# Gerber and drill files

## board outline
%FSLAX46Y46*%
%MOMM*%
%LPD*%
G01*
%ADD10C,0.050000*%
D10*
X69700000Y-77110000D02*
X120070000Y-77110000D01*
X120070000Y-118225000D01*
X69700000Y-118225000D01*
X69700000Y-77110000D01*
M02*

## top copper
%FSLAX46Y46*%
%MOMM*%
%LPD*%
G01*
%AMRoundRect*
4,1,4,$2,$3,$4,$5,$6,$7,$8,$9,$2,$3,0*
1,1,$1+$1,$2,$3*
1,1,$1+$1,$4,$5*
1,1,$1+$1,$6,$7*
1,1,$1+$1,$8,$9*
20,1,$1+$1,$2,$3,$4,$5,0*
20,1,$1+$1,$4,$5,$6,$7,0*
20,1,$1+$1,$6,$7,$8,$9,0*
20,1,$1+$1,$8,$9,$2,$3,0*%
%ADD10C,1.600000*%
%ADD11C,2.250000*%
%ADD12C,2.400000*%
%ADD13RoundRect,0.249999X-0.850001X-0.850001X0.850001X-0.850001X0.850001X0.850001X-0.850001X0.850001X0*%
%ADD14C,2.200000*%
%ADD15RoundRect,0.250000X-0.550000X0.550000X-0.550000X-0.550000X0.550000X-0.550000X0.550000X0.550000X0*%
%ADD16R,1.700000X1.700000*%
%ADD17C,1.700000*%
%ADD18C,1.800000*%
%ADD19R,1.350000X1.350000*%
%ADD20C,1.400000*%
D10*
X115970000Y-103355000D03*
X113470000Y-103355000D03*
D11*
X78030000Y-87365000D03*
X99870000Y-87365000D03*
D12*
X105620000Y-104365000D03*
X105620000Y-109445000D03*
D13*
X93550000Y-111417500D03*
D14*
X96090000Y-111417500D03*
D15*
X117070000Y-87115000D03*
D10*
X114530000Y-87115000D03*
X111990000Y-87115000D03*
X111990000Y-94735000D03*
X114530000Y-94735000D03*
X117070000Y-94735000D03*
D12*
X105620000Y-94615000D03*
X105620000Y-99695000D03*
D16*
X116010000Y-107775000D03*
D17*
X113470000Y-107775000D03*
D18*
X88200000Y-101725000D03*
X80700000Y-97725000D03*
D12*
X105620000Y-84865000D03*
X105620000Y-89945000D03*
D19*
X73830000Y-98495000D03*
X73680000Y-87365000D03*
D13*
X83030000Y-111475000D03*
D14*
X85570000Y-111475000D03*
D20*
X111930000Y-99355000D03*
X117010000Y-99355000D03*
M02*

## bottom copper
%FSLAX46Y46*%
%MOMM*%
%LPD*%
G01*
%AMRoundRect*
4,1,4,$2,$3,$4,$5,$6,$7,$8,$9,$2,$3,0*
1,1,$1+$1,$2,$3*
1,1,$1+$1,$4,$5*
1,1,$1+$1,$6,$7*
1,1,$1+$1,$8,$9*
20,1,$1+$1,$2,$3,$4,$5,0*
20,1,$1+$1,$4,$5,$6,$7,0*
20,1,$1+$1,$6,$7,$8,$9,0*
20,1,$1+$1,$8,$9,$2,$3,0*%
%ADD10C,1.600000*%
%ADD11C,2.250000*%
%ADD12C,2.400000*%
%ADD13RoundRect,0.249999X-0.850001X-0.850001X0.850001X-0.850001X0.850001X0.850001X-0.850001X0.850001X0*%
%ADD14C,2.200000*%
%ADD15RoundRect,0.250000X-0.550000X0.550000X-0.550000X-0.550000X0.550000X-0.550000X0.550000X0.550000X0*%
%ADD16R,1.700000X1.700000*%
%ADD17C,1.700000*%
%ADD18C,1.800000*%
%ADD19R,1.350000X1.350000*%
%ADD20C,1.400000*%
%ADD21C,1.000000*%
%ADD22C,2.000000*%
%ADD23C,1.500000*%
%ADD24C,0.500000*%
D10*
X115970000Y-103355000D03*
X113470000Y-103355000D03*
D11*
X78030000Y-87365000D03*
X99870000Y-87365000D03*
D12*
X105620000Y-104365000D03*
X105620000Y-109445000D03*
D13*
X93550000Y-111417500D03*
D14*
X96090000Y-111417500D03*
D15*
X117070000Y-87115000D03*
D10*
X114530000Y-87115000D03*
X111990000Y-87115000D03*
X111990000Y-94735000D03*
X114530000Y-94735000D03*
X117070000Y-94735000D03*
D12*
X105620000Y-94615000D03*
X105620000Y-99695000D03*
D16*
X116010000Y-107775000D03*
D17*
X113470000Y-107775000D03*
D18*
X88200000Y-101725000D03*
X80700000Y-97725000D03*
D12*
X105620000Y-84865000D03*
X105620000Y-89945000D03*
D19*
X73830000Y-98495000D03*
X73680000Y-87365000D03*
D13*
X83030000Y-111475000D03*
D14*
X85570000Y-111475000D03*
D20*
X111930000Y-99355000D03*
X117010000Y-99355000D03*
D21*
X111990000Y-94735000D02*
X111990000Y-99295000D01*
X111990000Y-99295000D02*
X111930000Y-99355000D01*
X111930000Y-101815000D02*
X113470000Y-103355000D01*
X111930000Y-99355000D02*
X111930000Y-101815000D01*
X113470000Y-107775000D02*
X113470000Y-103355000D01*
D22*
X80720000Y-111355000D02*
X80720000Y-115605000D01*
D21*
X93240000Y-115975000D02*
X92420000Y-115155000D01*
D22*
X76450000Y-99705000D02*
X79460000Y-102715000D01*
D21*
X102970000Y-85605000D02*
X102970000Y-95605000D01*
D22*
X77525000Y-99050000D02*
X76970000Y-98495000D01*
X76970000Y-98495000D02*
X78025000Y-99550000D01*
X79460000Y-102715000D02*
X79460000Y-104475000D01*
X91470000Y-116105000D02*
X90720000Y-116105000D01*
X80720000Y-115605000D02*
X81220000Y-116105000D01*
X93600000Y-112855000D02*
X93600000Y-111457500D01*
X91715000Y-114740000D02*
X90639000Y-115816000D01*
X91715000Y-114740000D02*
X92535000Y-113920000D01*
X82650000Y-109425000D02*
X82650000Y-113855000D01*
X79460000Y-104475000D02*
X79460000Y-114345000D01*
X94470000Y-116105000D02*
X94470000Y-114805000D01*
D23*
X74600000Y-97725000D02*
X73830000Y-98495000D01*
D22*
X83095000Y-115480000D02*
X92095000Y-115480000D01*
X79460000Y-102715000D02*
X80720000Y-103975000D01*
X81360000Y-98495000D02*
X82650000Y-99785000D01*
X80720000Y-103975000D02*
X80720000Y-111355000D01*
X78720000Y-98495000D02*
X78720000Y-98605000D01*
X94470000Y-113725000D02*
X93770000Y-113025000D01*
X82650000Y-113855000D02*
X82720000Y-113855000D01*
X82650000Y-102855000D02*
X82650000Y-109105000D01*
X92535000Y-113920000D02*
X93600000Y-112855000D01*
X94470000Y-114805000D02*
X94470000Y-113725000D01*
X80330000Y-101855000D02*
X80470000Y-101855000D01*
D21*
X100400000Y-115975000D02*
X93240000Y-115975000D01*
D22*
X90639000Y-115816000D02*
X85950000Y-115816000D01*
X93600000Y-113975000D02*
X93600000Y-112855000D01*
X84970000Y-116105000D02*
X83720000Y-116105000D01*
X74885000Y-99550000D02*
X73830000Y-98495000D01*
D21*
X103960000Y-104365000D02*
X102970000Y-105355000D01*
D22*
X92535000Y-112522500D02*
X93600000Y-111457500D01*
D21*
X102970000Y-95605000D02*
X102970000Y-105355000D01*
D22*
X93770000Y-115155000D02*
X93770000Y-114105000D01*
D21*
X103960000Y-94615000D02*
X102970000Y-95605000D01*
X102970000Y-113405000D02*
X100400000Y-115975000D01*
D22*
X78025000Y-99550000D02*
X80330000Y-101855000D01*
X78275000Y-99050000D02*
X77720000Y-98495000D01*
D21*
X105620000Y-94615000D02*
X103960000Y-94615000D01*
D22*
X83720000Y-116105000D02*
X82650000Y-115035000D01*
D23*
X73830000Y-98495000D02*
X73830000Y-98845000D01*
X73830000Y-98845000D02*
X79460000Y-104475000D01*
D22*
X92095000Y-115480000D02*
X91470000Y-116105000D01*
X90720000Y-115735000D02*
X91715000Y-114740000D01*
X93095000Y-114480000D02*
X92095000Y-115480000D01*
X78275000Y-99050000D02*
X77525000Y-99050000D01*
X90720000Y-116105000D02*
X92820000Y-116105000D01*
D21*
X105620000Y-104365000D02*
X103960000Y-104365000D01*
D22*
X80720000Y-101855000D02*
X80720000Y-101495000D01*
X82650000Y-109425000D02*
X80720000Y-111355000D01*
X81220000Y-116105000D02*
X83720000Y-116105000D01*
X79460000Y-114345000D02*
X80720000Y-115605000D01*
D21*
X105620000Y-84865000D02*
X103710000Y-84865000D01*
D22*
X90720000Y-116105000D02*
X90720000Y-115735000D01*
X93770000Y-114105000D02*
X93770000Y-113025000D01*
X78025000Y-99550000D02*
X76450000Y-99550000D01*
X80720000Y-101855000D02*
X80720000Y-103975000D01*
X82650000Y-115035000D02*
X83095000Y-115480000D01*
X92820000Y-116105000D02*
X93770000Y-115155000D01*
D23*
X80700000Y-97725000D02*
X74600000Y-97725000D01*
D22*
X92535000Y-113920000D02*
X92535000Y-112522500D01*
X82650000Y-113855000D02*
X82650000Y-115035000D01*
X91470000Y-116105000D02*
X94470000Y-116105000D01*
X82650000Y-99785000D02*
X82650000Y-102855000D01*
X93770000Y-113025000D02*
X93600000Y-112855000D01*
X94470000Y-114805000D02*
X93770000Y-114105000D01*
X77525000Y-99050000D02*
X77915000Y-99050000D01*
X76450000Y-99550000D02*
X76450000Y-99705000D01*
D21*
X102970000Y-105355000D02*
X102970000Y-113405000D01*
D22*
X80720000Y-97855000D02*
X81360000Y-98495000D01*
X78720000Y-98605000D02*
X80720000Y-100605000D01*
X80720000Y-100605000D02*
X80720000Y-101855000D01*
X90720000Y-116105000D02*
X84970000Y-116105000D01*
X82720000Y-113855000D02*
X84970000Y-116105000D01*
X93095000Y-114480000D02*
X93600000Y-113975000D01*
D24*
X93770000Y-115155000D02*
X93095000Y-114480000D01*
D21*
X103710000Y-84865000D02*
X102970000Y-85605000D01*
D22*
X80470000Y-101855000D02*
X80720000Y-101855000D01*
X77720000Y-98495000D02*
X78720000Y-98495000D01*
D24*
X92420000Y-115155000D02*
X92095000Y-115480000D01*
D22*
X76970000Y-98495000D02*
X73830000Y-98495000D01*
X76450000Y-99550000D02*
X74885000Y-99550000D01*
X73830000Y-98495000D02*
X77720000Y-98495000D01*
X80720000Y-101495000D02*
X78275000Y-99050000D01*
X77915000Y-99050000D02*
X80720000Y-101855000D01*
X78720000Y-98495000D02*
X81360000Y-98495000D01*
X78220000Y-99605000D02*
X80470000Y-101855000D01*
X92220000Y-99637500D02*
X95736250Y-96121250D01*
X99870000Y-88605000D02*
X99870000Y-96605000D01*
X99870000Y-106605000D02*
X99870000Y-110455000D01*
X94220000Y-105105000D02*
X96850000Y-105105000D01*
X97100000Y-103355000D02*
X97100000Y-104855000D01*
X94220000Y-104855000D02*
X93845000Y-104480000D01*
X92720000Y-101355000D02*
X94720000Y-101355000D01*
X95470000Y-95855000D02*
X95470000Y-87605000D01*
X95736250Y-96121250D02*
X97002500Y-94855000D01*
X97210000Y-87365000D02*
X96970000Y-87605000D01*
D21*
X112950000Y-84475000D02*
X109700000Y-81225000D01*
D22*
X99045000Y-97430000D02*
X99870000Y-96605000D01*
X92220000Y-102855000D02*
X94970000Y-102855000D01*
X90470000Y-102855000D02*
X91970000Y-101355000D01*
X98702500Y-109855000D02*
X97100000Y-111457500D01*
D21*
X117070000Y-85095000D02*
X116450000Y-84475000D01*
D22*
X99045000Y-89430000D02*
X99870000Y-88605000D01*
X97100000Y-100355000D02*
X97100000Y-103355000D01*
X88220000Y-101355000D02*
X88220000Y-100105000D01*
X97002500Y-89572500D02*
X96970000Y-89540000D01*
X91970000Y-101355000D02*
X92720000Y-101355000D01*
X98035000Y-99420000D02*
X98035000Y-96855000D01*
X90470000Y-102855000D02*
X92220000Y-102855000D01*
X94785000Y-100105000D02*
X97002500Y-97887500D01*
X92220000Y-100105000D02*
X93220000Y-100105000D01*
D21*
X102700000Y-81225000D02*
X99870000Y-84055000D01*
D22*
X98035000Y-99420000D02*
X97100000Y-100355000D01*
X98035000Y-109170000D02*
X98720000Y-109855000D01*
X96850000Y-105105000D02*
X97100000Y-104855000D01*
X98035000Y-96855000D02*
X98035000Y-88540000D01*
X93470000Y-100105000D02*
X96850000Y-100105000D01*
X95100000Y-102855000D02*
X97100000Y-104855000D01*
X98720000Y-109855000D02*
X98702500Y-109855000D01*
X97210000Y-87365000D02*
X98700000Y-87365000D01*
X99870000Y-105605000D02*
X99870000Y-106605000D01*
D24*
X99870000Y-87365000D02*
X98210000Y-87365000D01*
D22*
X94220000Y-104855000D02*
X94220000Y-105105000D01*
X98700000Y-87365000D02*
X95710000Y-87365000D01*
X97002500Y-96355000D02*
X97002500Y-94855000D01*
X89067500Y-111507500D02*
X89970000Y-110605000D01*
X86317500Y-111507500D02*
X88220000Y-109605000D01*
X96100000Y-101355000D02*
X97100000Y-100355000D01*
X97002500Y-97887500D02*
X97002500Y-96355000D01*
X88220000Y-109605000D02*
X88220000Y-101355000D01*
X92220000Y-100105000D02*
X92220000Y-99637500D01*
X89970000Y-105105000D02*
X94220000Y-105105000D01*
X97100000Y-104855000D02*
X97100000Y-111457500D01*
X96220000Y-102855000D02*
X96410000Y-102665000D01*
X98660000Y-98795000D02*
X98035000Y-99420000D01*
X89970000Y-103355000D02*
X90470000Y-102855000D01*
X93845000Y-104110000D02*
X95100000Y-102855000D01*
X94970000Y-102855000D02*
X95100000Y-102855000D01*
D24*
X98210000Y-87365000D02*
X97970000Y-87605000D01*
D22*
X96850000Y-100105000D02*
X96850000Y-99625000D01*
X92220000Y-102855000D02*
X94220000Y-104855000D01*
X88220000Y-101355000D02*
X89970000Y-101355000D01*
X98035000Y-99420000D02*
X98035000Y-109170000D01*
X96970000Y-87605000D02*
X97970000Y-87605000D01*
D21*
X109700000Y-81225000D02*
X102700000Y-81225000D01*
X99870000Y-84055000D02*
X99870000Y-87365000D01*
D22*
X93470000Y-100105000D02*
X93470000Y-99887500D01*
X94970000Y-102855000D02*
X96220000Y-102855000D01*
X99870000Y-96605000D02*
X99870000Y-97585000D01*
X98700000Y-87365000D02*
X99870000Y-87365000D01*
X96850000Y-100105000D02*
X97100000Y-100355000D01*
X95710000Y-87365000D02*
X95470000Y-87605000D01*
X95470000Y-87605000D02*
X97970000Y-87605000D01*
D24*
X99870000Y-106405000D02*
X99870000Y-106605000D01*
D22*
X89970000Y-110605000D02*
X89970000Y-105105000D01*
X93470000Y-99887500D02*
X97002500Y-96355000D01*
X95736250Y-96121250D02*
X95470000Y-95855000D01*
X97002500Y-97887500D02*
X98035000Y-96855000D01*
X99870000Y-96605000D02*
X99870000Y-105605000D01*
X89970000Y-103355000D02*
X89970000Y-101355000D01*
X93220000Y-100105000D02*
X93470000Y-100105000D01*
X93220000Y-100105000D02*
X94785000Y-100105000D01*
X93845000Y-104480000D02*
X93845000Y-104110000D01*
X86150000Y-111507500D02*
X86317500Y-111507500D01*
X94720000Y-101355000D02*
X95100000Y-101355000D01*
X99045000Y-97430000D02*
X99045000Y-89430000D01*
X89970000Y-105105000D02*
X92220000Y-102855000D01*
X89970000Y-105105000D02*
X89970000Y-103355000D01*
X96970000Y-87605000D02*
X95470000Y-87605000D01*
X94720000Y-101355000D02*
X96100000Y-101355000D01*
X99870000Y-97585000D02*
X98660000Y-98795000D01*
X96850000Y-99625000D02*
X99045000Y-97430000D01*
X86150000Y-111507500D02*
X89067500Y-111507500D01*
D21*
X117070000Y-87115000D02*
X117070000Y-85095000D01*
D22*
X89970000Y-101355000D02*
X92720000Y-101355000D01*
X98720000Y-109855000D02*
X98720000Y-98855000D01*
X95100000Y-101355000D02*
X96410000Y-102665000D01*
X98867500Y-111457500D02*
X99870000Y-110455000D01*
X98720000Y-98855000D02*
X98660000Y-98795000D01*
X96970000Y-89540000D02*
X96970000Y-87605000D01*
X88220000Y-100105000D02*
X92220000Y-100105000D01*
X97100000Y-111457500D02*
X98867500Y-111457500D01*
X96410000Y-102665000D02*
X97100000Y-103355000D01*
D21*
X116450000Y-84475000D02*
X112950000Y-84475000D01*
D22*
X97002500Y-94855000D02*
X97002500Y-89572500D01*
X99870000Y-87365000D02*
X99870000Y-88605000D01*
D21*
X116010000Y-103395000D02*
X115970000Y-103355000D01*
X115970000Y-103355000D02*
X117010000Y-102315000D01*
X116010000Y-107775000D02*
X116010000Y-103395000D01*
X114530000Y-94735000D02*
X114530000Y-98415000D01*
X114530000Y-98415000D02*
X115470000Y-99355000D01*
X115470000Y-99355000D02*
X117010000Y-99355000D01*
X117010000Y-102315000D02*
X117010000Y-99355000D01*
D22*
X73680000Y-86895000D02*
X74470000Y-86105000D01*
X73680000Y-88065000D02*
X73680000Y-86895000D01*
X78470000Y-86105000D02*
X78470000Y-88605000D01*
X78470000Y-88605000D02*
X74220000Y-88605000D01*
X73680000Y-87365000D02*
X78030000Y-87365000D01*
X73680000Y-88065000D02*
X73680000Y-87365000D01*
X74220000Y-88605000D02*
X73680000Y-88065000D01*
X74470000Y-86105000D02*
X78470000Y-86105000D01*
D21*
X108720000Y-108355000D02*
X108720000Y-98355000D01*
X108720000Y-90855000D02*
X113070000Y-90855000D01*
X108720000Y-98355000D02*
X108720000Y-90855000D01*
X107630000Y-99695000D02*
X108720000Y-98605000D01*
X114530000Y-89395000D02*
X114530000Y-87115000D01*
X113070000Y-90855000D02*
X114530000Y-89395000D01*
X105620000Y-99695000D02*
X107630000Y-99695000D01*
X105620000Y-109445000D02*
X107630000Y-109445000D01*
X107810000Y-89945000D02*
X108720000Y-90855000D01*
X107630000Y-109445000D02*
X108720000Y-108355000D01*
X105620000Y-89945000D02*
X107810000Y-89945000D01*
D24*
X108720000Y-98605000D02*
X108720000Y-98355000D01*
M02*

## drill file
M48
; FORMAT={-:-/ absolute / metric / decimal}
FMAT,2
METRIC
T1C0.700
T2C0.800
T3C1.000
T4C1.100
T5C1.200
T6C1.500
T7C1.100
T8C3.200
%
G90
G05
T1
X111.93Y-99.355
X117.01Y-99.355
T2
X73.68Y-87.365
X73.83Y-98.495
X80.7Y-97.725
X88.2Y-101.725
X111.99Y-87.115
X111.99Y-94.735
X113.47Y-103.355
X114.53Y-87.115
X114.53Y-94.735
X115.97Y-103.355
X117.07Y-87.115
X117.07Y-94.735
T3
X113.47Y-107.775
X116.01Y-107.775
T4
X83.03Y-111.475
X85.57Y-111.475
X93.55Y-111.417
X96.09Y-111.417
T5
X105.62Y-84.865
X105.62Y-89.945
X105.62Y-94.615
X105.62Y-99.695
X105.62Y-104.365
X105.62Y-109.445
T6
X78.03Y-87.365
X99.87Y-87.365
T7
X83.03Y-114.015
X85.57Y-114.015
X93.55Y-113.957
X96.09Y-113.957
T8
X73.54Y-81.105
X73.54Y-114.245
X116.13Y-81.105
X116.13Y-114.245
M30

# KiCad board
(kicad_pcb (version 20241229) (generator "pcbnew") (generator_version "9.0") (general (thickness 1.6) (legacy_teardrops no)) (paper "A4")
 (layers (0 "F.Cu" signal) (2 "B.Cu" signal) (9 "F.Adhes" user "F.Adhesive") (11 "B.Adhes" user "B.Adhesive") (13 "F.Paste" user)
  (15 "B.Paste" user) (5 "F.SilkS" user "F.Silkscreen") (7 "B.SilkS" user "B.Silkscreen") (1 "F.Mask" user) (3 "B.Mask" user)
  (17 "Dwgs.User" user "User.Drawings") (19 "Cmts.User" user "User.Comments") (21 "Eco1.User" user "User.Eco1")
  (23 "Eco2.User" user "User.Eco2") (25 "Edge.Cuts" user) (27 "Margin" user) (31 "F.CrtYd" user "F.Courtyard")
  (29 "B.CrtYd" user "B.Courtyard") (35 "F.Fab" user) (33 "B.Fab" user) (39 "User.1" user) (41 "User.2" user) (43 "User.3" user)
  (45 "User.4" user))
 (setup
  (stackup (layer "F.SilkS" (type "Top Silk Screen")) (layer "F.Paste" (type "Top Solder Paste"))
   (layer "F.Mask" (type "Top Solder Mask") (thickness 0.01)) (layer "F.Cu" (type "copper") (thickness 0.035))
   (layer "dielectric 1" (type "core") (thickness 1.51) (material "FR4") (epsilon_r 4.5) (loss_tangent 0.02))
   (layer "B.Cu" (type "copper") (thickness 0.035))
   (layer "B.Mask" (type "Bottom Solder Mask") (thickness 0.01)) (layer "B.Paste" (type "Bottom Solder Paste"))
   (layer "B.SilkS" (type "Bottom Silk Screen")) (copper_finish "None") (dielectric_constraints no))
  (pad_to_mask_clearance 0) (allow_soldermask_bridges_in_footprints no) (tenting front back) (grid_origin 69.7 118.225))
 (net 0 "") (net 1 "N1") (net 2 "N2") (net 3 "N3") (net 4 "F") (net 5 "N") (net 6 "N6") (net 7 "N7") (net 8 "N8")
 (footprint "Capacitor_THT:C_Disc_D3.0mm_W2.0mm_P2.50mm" (layer "F.Cu") (at 115.97 103.355 180)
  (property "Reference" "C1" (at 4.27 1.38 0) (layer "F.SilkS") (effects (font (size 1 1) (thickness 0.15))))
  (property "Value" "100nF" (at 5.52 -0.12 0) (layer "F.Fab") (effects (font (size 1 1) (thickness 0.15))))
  (pad "1" thru_hole circle (at 0 0 180) (size 1.6 1.6) (drill 0.8) (layers "*.Cu" "*.Mask") (remove_unused_layers no) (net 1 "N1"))
  (pad "2" thru_hole circle (at 2.5 0 180) (size 1.6 1.6) (drill 0.8) (layers "*.Cu" "*.Mask") (remove_unused_layers no) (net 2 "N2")))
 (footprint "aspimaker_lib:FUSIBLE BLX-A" (layer "F.Cu") (at 88.95 87.365)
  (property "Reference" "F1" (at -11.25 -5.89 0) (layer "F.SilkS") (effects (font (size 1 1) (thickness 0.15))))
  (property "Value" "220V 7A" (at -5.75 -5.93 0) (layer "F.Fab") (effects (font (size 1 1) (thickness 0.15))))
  (pad "1" thru_hole circle (at -10.92 0) (size 2.25 2.25) (drill 1.5) (layers "*.Cu" "*.Mask") (remove_unused_layers no) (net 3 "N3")
   (solder_mask_margin 0.102))
  (pad "2" thru_hole circle (at 10.92 0) (size 2.25 2.25) (drill 1.5) (layers "*.Cu" "*.Mask") (remove_unused_layers no) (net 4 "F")
   (solder_mask_margin 0.102)))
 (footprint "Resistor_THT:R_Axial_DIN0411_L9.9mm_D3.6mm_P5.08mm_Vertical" (layer "F.Cu") (at 105.62 104.365 -90)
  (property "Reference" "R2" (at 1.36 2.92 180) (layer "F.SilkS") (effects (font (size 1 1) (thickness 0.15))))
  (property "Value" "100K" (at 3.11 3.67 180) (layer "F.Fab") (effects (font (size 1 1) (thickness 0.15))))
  (pad "1" thru_hole circle (at 0 0 270) (size 2.4 2.4) (drill 1.2) (layers "*.Cu" "*.Mask") (remove_unused_layers no) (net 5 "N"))
  (pad "2" thru_hole circle (at 5.08 0 270) (size 2.4 2.4) (drill 1.2) (layers "*.Cu" "*.Mask") (remove_unused_layers no) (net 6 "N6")))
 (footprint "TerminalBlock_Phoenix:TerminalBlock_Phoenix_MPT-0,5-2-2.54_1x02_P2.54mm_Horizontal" (layer "F.Cu") (at 93.55 111.4175)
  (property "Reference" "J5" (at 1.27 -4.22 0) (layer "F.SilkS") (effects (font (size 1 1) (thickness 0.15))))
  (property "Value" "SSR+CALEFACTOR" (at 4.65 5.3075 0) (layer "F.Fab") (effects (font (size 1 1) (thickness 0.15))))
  (pad "" np_thru_hole circle (at 0 2.54) (size 1.1 1.1) (drill 1.1) (layers "*.Cu" "*.Mask"))
  (pad "" np_thru_hole circle (at 2.54 2.54) (size 1.1 1.1) (drill 1.1) (layers "*.Cu" "*.Mask"))
  (pad "1" thru_hole roundrect (at 0 0) (size 2.2 2.2) (drill 1.1) (layers "*.Cu" "*.Mask") (remove_unused_layers no)
   (roundrect_rratio 0.113636) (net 5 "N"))
  (pad "2" thru_hole circle (at 2.54 0) (size 2.2 2.2) (drill 1.1) (layers "*.Cu" "*.Mask") (remove_unused_layers no) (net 4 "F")))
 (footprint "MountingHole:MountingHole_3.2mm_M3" (layer "F.Cu") (at 116.13 114.245)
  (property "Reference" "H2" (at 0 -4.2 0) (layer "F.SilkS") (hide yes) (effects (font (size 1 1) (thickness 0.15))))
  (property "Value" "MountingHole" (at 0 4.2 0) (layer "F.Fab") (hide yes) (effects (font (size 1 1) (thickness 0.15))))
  (pad "" np_thru_hole circle (at 0 0) (size 3.2 3.2) (drill 3.2) (layers "*.Cu" "*.Mask")))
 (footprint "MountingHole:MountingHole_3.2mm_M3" (layer "F.Cu") (at 73.54 81.105)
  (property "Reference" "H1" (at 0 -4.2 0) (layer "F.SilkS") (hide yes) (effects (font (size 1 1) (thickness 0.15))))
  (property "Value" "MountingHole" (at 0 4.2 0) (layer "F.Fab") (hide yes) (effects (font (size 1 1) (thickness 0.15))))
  (pad "" np_thru_hole circle (at 0 0) (size 3.2 3.2) (drill 3.2) (layers "*.Cu" "*.Mask")))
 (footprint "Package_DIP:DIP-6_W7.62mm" (layer "F.Cu") (at 117.07 87.115 -90)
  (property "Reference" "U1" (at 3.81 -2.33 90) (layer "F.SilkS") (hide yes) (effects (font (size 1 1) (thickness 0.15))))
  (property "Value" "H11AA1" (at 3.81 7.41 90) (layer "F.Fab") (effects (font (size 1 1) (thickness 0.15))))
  (pad "1" thru_hole roundrect (at 0 0 270) (size 1.6 1.6) (drill 0.8) (layers "*.Cu" "*.Mask") (remove_unused_layers no)
   (roundrect_rratio 0.15625) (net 4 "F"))
  (pad "2" thru_hole circle (at 0 2.54 270) (size 1.6 1.6) (drill 0.8) (layers "*.Cu" "*.Mask") (remove_unused_layers no) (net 6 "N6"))
  (pad "3" thru_hole circle (at 0 5.08 270) (size 1.6 1.6) (drill 0.8) (layers "*.Cu" "*.Mask") (remove_unused_layers no) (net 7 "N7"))
  (pad "4" thru_hole circle (at 7.62 5.08 270) (size 1.6 1.6) (drill 0.8) (layers "*.Cu" "*.Mask") (remove_unused_layers no) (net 2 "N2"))
  (pad "5" thru_hole circle (at 7.62 2.54 270) (size 1.6 1.6) (drill 0.8) (layers "*.Cu" "*.Mask") (remove_unused_layers no) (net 1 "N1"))
  (pad "6" thru_hole circle (at 7.62 0 270) (size 1.6 1.6) (drill 0.8) (layers "*.Cu" "*.Mask") (remove_unused_layers no) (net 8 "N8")))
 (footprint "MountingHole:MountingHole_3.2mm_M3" (layer "F.Cu") (at 116.13 81.105)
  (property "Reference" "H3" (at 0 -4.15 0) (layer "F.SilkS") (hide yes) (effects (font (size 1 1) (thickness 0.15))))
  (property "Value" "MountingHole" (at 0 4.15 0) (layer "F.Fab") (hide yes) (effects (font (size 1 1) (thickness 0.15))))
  (pad "" np_thru_hole circle (at 0 0) (size 3.2 3.2) (drill 3.2) (layers "*.Cu" "*.Mask")))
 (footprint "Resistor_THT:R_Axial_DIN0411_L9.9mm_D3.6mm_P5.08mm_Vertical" (layer "F.Cu") (at 105.62 94.615 -90)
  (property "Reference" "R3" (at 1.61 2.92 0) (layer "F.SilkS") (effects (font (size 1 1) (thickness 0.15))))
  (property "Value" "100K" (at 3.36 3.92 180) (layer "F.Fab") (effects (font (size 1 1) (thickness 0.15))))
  (pad "1" thru_hole circle (at 0 0 270) (size 2.4 2.4) (drill 1.2) (layers "*.Cu" "*.Mask") (remove_unused_layers no) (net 5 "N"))
  (pad "2" thru_hole circle (at 5.08 0 270) (size 2.4 2.4) (drill 1.2) (layers "*.Cu" "*.Mask") (remove_unused_layers no) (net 6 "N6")))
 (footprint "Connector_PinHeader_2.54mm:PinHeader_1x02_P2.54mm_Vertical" (layer "F.Cu") (at 116.01 107.775 -90)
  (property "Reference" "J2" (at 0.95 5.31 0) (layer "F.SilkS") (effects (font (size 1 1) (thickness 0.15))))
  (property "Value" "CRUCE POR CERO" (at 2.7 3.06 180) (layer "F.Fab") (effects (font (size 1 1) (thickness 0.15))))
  (pad "1" thru_hole rect (at 0 0 270) (size 1.7 1.7) (drill 1) (layers "*.Cu" "*.Mask") (remove_unused_layers no) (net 1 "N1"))
  (pad "2" thru_hole circle (at 0 2.54 270) (size 1.7 1.7) (drill 1) (layers "*.Cu" "*.Mask") (remove_unused_layers no) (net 2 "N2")))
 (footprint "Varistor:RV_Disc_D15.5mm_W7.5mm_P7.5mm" (layer "F.Cu") (at 88.2 101.725 180)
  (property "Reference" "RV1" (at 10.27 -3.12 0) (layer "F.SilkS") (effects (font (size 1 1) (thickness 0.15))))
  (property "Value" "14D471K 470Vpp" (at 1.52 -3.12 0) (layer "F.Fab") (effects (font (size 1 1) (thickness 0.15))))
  (pad "1" thru_hole circle (at 0 0 180) (size 1.8 1.8) (drill 0.8) (layers "*.Cu" "*.Mask") (remove_unused_layers no) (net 4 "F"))
  (pad "2" thru_hole circle (at 7.5 4 180) (size 1.8 1.8) (drill 0.8) (layers "*.Cu" "*.Mask") (remove_unused_layers no) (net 5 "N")))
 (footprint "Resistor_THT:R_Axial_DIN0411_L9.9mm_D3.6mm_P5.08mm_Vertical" (layer "F.Cu") (at 105.62 84.865 -90)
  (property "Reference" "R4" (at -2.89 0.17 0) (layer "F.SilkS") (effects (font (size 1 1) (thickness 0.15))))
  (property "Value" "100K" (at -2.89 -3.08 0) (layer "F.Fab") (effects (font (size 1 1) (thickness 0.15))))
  (pad "1" thru_hole circle (at 0 0 270) (size 2.4 2.4) (drill 1.2) (layers "*.Cu" "*.Mask") (remove_unused_layers no) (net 5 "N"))
  (pad "2" thru_hole circle (at 5.08 0 270) (size 2.4 2.4) (drill 1.2) (layers "*.Cu" "*.Mask") (remove_unused_layers no) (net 6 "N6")))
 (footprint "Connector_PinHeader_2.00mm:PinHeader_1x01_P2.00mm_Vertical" (layer "F.Cu") (at 73.83 98.495)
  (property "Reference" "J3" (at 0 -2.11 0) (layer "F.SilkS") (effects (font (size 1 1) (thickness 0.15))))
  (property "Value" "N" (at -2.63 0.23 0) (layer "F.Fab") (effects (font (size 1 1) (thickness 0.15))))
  (pad "1" thru_hole rect (at 0 0) (size 1.35 1.35) (drill 0.8) (layers "*.Cu" "*.Mask") (remove_unused_layers no) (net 5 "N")))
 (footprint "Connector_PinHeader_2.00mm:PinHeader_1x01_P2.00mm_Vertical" (layer "F.Cu") (at 73.68 87.365)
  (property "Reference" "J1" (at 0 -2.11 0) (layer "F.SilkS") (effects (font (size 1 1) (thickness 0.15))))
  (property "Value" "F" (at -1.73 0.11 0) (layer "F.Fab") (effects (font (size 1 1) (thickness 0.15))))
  (pad "1" thru_hole rect (at 0 0) (size 1.35 1.35) (drill 0.8) (layers "*.Cu" "*.Mask") (remove_unused_layers no) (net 3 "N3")))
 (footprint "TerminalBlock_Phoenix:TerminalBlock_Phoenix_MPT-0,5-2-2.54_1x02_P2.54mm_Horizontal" (layer "F.Cu") (at 83.03 111.475)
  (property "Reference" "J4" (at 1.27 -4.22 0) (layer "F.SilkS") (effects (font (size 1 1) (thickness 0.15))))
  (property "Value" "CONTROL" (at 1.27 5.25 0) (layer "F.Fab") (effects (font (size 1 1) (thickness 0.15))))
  (pad "" np_thru_hole circle (at 0 2.54) (size 1.1 1.1) (drill 1.1) (layers "*.Cu" "*.Mask"))
  (pad "" np_thru_hole circle (at 2.54 2.54) (size 1.1 1.1) (drill 1.1) (layers "*.Cu" "*.Mask"))
  (pad "1" thru_hole roundrect (at 0 0) (size 2.2 2.2) (drill 1.1) (layers "*.Cu" "*.Mask") (remove_unused_layers no)
   (roundrect_rratio 0.113636) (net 5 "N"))
  (pad "2" thru_hole circle (at 2.54 0) (size 2.2 2.2) (drill 1.1) (layers "*.Cu" "*.Mask") (remove_unused_layers no) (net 4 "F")))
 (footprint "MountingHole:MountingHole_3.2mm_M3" (layer "F.Cu") (at 73.54 114.245)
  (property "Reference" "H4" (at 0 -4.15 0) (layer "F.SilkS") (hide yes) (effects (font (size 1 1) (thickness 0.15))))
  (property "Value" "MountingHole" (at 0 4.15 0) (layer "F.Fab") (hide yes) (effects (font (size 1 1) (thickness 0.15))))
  (pad "" np_thru_hole circle (at 0 0) (size 3.2 3.2) (drill 3.2) (layers "*.Cu" "*.Mask")))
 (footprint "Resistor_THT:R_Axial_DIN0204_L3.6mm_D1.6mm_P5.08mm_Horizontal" (layer "F.Cu") (at 111.93 99.355)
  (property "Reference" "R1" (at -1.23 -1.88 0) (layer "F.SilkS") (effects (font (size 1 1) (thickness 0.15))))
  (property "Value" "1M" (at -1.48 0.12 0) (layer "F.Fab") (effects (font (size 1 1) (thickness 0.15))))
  (pad "1" thru_hole circle (at 0 0) (size 1.4 1.4) (drill 0.7) (layers "*.Cu" "*.Mask") (remove_unused_layers no) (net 2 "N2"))
  (pad "2" thru_hole circle (at 5.08 0) (size 1.4 1.4) (drill 0.7) (layers "*.Cu" "*.Mask") (remove_unused_layers no) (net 1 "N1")))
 (gr_rect (start 69.7 77.11) (end 120.07 118.225) (stroke (width 0.05) (type solid)) (fill no) (layer "Edge.Cuts"))
 (segment (start 111.99 94.735) (end 111.99 99.295) (width 1) (layer "B.Cu") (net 2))
 (segment (start 111.99 99.295) (end 111.93 99.355) (width 1) (layer "B.Cu") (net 2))
 (segment (start 111.93 101.815) (end 113.47 103.355) (width 1) (layer "B.Cu") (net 2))
 (segment (start 111.93 99.355) (end 111.93 101.815) (width 1) (layer "B.Cu") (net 2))
 (segment (start 113.47 107.775) (end 113.47 103.355) (width 1) (layer "B.Cu") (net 2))
 (segment (start 80.72 111.355) (end 80.72 115.605) (width 2) (layer "B.Cu") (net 5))
 (segment (start 93.24 115.975) (end 92.42 115.155) (width 1) (layer "B.Cu") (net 5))
 (segment (start 76.45 99.705) (end 79.46 102.715) (width 2) (layer "B.Cu") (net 5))
 (segment (start 102.97 85.605) (end 102.97 95.605) (width 1) (layer "B.Cu") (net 5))
 (segment (start 77.525 99.05) (end 76.97 98.495) (width 2) (layer "B.Cu") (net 5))
 (segment (start 76.97 98.495) (end 78.025 99.55) (width 2) (layer "B.Cu") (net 5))
 (segment (start 79.46 102.715) (end 79.46 104.475) (width 2) (layer "B.Cu") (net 5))
 (segment (start 91.47 116.105) (end 90.72 116.105) (width 2) (layer "B.Cu") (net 5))
 (segment (start 80.72 115.605) (end 81.22 116.105) (width 2) (layer "B.Cu") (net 5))
 (segment (start 93.6 112.855) (end 93.6 111.4575) (width 2) (layer "B.Cu") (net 5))
 (segment (start 91.715 114.74) (end 90.639 115.816) (width 2) (layer "B.Cu") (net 5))
 (segment (start 91.715 114.74) (end 92.535 113.92) (width 2) (layer "B.Cu") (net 5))
 (segment (start 82.65 109.425) (end 82.65 113.855) (width 2) (layer "B.Cu") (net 5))
 (segment (start 79.46 104.475) (end 79.46 114.345) (width 2) (layer "B.Cu") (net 5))
 (segment (start 94.47 116.105) (end 94.47 114.805) (width 2) (layer "B.Cu") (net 5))
 (segment (start 74.6 97.725) (end 73.83 98.495) (width 1.5) (layer "B.Cu") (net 5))
 (segment (start 83.095 115.48) (end 92.095 115.48) (width 2) (layer "B.Cu") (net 5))
 (segment (start 79.46 102.715) (end 80.72 103.975) (width 2) (layer "B.Cu") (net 5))
 (segment (start 81.36 98.495) (end 82.65 99.785) (width 2) (layer "B.Cu") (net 5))
 (segment (start 80.72 103.975) (end 80.72 111.355) (width 2) (layer "B.Cu") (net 5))
 (segment (start 78.72 98.495) (end 78.72 98.605) (width 2) (layer "B.Cu") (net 5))
 (segment (start 94.47 113.725) (end 93.77 113.025) (width 2) (layer "B.Cu") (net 5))
 (segment (start 82.65 113.855) (end 82.72 113.855) (width 2) (layer "B.Cu") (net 5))
 (segment (start 82.65 102.855) (end 82.65 109.105) (width 2) (layer "B.Cu") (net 5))
 (segment (start 92.535 113.92) (end 93.6 112.855) (width 2) (layer "B.Cu") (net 5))
 (segment (start 94.47 114.805) (end 94.47 113.725) (width 2) (layer "B.Cu") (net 5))
 (segment (start 80.33 101.855) (end 80.47 101.855) (width 2) (layer "B.Cu") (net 5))
 (segment (start 100.4 115.975) (end 93.24 115.975) (width 1) (layer "B.Cu") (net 5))
 (segment (start 90.639 115.816) (end 85.95 115.816) (width 2) (layer "B.Cu") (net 5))
 (segment (start 93.6 113.975) (end 93.6 112.855) (width 2) (layer "B.Cu") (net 5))
 (segment (start 84.97 116.105) (end 83.72 116.105) (width 2) (layer "B.Cu") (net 5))
 (segment (start 74.885 99.55) (end 73.83 98.495) (width 2) (layer "B.Cu") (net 5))
 (segment (start 103.96 104.365) (end 102.97 105.355) (width 1) (layer "B.Cu") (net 5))
 (segment (start 92.535 112.5225) (end 93.6 111.4575) (width 2) (layer "B.Cu") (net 5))
 (segment (start 102.97 95.605) (end 102.97 105.355) (width 1) (layer "B.Cu") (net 5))
 (segment (start 93.77 115.155) (end 93.77 114.105) (width 2) (layer "B.Cu") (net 5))
 (segment (start 103.96 94.615) (end 102.97 95.605) (width 1) (layer "B.Cu") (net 5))
 (segment (start 102.97 113.405) (end 100.4 115.975) (width 1) (layer "B.Cu") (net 5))
 (segment (start 78.025 99.55) (end 80.33 101.855) (width 2) (layer "B.Cu") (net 5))
 (segment (start 78.275 99.05) (end 77.72 98.495) (width 2) (layer "B.Cu") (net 5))
 (segment (start 105.62 94.615) (end 103.96 94.615) (width 1) (layer "B.Cu") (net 5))
 (segment (start 83.72 116.105) (end 82.65 115.035) (width 2) (layer "B.Cu") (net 5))
 (segment (start 73.83 98.495) (end 73.83 98.845) (width 1.5) (layer "B.Cu") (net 5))
 (segment (start 73.83 98.845) (end 79.46 104.475) (width 1.5) (layer "B.Cu") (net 5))
 (segment (start 92.095 115.48) (end 91.47 116.105) (width 2) (layer "B.Cu") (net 5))
 (segment (start 90.72 115.735) (end 91.715 114.74) (width 2) (layer "B.Cu") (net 5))
 (segment (start 93.095 114.48) (end 92.095 115.48) (width 2) (layer "B.Cu") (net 5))
 (segment (start 78.275 99.05) (end 77.525 99.05) (width 2) (layer "B.Cu") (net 5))
 (segment (start 90.72 116.105) (end 92.82 116.105) (width 2) (layer "B.Cu") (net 5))
 (segment (start 105.62 104.365) (end 103.96 104.365) (width 1) (layer "B.Cu") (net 5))
 (segment (start 80.72 101.855) (end 80.72 101.495) (width 2) (layer "B.Cu") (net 5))
 (segment (start 82.65 109.425) (end 80.72 111.355) (width 2) (layer "B.Cu") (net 5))
 (segment (start 81.22 116.105) (end 83.72 116.105) (width 2) (layer "B.Cu") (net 5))
 (segment (start 79.46 114.345) (end 80.72 115.605) (width 2) (layer "B.Cu") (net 5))
 (segment (start 105.62 84.865) (end 103.71 84.865) (width 1) (layer "B.Cu") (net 5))
 (segment (start 90.72 116.105) (end 90.72 115.735) (width 2) (layer "B.Cu") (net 5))
 (segment (start 93.77 114.105) (end 93.77 113.025) (width 2) (layer "B.Cu") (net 5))
 (segment (start 78.025 99.55) (end 76.45 99.55) (width 2) (layer "B.Cu") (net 5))
 (segment (start 80.72 101.855) (end 80.72 103.975) (width 2) (layer "B.Cu") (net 5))
 (segment (start 82.65 115.035) (end 83.095 115.48) (width 2) (layer "B.Cu") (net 5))
 (segment (start 92.82 116.105) (end 93.77 115.155) (width 2) (layer "B.Cu") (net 5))
 (segment (start 80.7 97.725) (end 74.6 97.725) (width 1.5) (layer "B.Cu") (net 5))
 (segment (start 92.535 113.92) (end 92.535 112.5225) (width 2) (layer "B.Cu") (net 5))
 (segment (start 82.65 113.855) (end 82.65 115.035) (width 2) (layer "B.Cu") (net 5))
 (segment (start 91.47 116.105) (end 94.47 116.105) (width 2) (layer "B.Cu") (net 5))
 (segment (start 82.65 99.785) (end 82.65 102.855) (width 2) (layer "B.Cu") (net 5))
 (segment (start 93.77 113.025) (end 93.6 112.855) (width 2) (layer "B.Cu") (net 5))
 (segment (start 94.47 114.805) (end 93.77 114.105) (width 2) (layer "B.Cu") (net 5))
 (segment (start 77.525 99.05) (end 77.915 99.05) (width 2) (layer "B.Cu") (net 5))
 (segment (start 76.45 99.55) (end 76.45 99.705) (width 2) (layer "B.Cu") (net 5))
 (segment (start 102.97 105.355) (end 102.97 113.405) (width 1) (layer "B.Cu") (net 5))
 (segment (start 80.72 97.855) (end 81.36 98.495) (width 2) (layer "B.Cu") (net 5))
 (segment (start 78.72 98.605) (end 80.72 100.605) (width 2) (layer "B.Cu") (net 5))
 (segment (start 80.72 100.605) (end 80.72 101.855) (width 2) (layer "B.Cu") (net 5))
 (segment (start 90.72 116.105) (end 84.97 116.105) (width 2) (layer "B.Cu") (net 5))
 (segment (start 82.72 113.855) (end 84.97 116.105) (width 2) (layer "B.Cu") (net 5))
 (segment (start 93.095 114.48) (end 93.6 113.975) (width 2) (layer "B.Cu") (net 5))
 (segment (start 93.77 115.155) (end 93.095 114.48) (width 0.5) (layer "B.Cu") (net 5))
 (segment (start 103.71 84.865) (end 102.97 85.605) (width 1) (layer "B.Cu") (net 5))
 (segment (start 80.47 101.855) (end 80.72 101.855) (width 2) (layer "B.Cu") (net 5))
 (segment (start 77.72 98.495) (end 78.72 98.495) (width 2) (layer "B.Cu") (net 5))
 (segment (start 92.42 115.155) (end 92.095 115.48) (width 0.5) (layer "B.Cu") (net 5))
 (segment (start 76.97 98.495) (end 73.83 98.495) (width 2) (layer "B.Cu") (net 5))
 (segment (start 76.45 99.55) (end 74.885 99.55) (width 2) (layer "B.Cu") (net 5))
 (segment (start 73.83 98.495) (end 77.72 98.495) (width 2) (layer "B.Cu") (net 5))
 (segment (start 80.72 101.495) (end 78.275 99.05) (width 2) (layer "B.Cu") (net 5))
 (segment (start 77.915 99.05) (end 80.72 101.855) (width 2) (layer "B.Cu") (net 5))
 (segment (start 78.72 98.495) (end 81.36 98.495) (width 2) (layer "B.Cu") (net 5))
 (segment (start 78.22 99.605) (end 80.47 101.855) (width 2) (layer "B.Cu") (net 5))
 (segment (start 92.22 99.6375) (end 95.73625 96.12125) (width 2) (layer "B.Cu") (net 4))
 (segment (start 99.87 88.605) (end 99.87 96.605) (width 2) (layer "B.Cu") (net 4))
 (segment (start 99.87 106.605) (end 99.87 110.455) (width 2) (layer "B.Cu") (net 4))
 (segment (start 94.22 105.105) (end 96.85 105.105) (width 2) (layer "B.Cu") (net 4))
 (segment (start 97.1 103.355) (end 97.1 104.855) (width 2) (layer "B.Cu") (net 4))
 (segment (start 94.22 104.855) (end 93.845 104.48) (width 2) (layer "B.Cu") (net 4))
 (segment (start 92.72 101.355) (end 94.72 101.355) (width 2) (layer "B.Cu") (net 4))
 (segment (start 95.47 95.855) (end 95.47 87.605) (width 2) (layer "B.Cu") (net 4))
 (segment (start 95.73625 96.12125) (end 97.0025 94.855) (width 2) (layer "B.Cu") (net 4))
 (segment (start 97.21 87.365) (end 96.97 87.605) (width 2) (layer "B.Cu") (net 4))
 (segment (start 112.95 84.475) (end 109.7 81.225) (width 1) (layer "B.Cu") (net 4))
 (segment (start 99.045 97.43) (end 99.87 96.605) (width 2) (layer "B.Cu") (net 4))
 (segment (start 92.22 102.855) (end 94.97 102.855) (width 2) (layer "B.Cu") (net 4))
 (segment (start 90.47 102.855) (end 91.97 101.355) (width 2) (layer "B.Cu") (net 4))
 (segment (start 98.7025 109.855) (end 97.1 111.4575) (width 2) (layer "B.Cu") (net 4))
 (segment (start 117.07 85.095) (end 116.45 84.475) (width 1) (layer "B.Cu") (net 4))
 (segment (start 99.045 89.43) (end 99.87 88.605) (width 2) (layer "B.Cu") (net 4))
 (segment (start 97.1 100.355) (end 97.1 103.355) (width 2) (layer "B.Cu") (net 4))
 (segment (start 88.22 101.355) (end 88.22 100.105) (width 2) (layer "B.Cu") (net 4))
 (segment (start 97.0025 89.5725) (end 96.97 89.54) (width 2) (layer "B.Cu") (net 4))
 (segment (start 91.97 101.355) (end 92.72 101.355) (width 2) (layer "B.Cu") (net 4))
 (segment (start 98.035 99.42) (end 98.035 96.855) (width 2) (layer "B.Cu") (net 4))
 (segment (start 90.47 102.855) (end 92.22 102.855) (width 2) (layer "B.Cu") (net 4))
 (segment (start 94.785 100.105) (end 97.0025 97.8875) (width 2) (layer "B.Cu") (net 4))
 (segment (start 92.22 100.105) (end 93.22 100.105) (width 2) (layer "B.Cu") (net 4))
 (segment (start 102.7 81.225) (end 99.87 84.055) (width 1) (layer "B.Cu") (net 4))
 (segment (start 98.035 99.42) (end 97.1 100.355) (width 2) (layer "B.Cu") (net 4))
 (segment (start 98.035 109.17) (end 98.72 109.855) (width 2) (layer "B.Cu") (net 4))
 (segment (start 96.85 105.105) (end 97.1 104.855) (width 2) (layer "B.Cu") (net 4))
 (segment (start 98.035 96.855) (end 98.035 88.54) (width 2) (layer "B.Cu") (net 4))
 (segment (start 93.47 100.105) (end 96.85 100.105) (width 2) (layer "B.Cu") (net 4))
 (segment (start 95.1 102.855) (end 97.1 104.855) (width 2) (layer "B.Cu") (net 4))
 (segment (start 98.72 109.855) (end 98.7025 109.855) (width 2) (layer "B.Cu") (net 4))
 (segment (start 97.21 87.365) (end 98.7 87.365) (width 2) (layer "B.Cu") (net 4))
 (segment (start 99.87 105.605) (end 99.87 106.605) (width 2) (layer "B.Cu") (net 4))
 (segment (start 99.87 87.365) (end 98.21 87.365) (width 0.5) (layer "B.Cu") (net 4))
 (segment (start 94.22 104.855) (end 94.22 105.105) (width 2) (layer "B.Cu") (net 4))
 (segment (start 98.7 87.365) (end 95.71 87.365) (width 2) (layer "B.Cu") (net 4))
 (segment (start 97.0025 96.355) (end 97.0025 94.855) (width 2) (layer "B.Cu") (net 4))
 (segment (start 89.0675 111.5075) (end 89.97 110.605) (width 2) (layer "B.Cu") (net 4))
 (segment (start 86.3175 111.5075) (end 88.22 109.605) (width 2) (layer "B.Cu") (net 4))
 (segment (start 96.1 101.355) (end 97.1 100.355) (width 2) (layer "B.Cu") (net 4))
 (segment (start 97.0025 97.8875) (end 97.0025 96.355) (width 2) (layer "B.Cu") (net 4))
 (segment (start 88.22 109.605) (end 88.22 101.355) (width 2) (layer "B.Cu") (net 4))
 (segment (start 92.22 100.105) (end 92.22 99.6375) (width 2) (layer "B.Cu") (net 4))
 (segment (start 89.97 105.105) (end 94.22 105.105) (width 2) (layer "B.Cu") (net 4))
 (segment (start 97.1 104.855) (end 97.1 111.4575) (width 2) (layer "B.Cu") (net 4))
 (segment (start 96.22 102.855) (end 96.41 102.665) (width 2) (layer "B.Cu") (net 4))
 (segment (start 98.66 98.795) (end 98.035 99.42) (width 2) (layer "B.Cu") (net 4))
 (segment (start 89.97 103.355) (end 90.47 102.855) (width 2) (layer "B.Cu") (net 4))
 (segment (start 93.845 104.11) (end 95.1 102.855) (width 2) (layer "B.Cu") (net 4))
 (segment (start 94.97 102.855) (end 95.1 102.855) (width 2) (layer "B.Cu") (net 4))
 (segment (start 98.21 87.365) (end 97.97 87.605) (width 0.5) (layer "B.Cu") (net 4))
 (segment (start 96.85 100.105) (end 96.85 99.625) (width 2) (layer "B.Cu") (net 4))
 (segment (start 92.22 102.855) (end 94.22 104.855) (width 2) (layer "B.Cu") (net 4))
 (segment (start 88.22 101.355) (end 89.97 101.355) (width 2) (layer "B.Cu") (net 4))
 (segment (start 98.035 99.42) (end 98.035 109.17) (width 2) (layer "B.Cu") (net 4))
 (segment (start 96.97 87.605) (end 97.97 87.605) (width 2) (layer "B.Cu") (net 4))
 (segment (start 109.7 81.225) (end 102.7 81.225) (width 1) (layer "B.Cu") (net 4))
 (segment (start 99.87 84.055) (end 99.87 87.365) (width 1) (layer "B.Cu") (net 4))
 (segment (start 93.47 100.105) (end 93.47 99.8875) (width 2) (layer "B.Cu") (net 4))
 (segment (start 94.97 102.855) (end 96.22 102.855) (width 2) (layer "B.Cu") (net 4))
 (segment (start 99.87 96.605) (end 99.87 97.585) (width 2) (layer "B.Cu") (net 4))
 (segment (start 98.7 87.365) (end 99.87 87.365) (width 2) (layer "B.Cu") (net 4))
 (segment (start 96.85 100.105) (end 97.1 100.355) (width 2) (layer "B.Cu") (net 4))
 (segment (start 95.71 87.365) (end 95.47 87.605) (width 2) (layer "B.Cu") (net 4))
 (segment (start 95.47 87.605) (end 97.97 87.605) (width 2) (layer "B.Cu") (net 4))
 (segment (start 99.87 106.405) (end 99.87 106.605) (width 0.5) (layer "B.Cu") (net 4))
 (segment (start 89.97 110.605) (end 89.97 105.105) (width 2) (layer "B.Cu") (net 4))
 (segment (start 93.47 99.8875) (end 97.0025 96.355) (width 2) (layer "B.Cu") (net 4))
 (segment (start 95.73625 96.12125) (end 95.47 95.855) (width 2) (layer "B.Cu") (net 4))
 (segment (start 97.0025 97.8875) (end 98.035 96.855) (width 2) (layer "B.Cu") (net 4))
 (segment (start 99.87 96.605) (end 99.87 105.605) (width 2) (layer "B.Cu") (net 4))
 (segment (start 89.97 103.355) (end 89.97 101.355) (width 2) (layer "B.Cu") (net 4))
 (segment (start 93.22 100.105) (end 93.47 100.105) (width 2) (layer "B.Cu") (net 4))
 (segment (start 93.22 100.105) (end 94.785 100.105) (width 2) (layer "B.Cu") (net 4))
 (segment (start 93.845 104.48) (end 93.845 104.11) (width 2) (layer "B.Cu") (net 4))
 (segment (start 86.15 111.5075) (end 86.3175 111.5075) (width 2) (layer "B.Cu") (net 4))
 (segment (start 94.72 101.355) (end 95.1 101.355) (width 2) (layer "B.Cu") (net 4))
 (segment (start 99.045 97.43) (end 99.045 89.43) (width 2) (layer "B.Cu") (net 4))
 (segment (start 89.97 105.105) (end 92.22 102.855) (width 2) (layer "B.Cu") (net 4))
 (segment (start 89.97 105.105) (end 89.97 103.355) (width 2) (layer "B.Cu") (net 4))
 (segment (start 96.97 87.605) (end 95.47 87.605) (width 2) (layer "B.Cu") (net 4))
 (segment (start 94.72 101.355) (end 96.1 101.355) (width 2) (layer "B.Cu") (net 4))
 (segment (start 99.87 97.585) (end 98.66 98.795) (width 2) (layer "B.Cu") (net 4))
 (segment (start 96.85 99.625) (end 99.045 97.43) (width 2) (layer "B.Cu") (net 4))
 (segment (start 86.15 111.5075) (end 89.0675 111.5075) (width 2) (layer "B.Cu") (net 4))
 (segment (start 117.07 87.115) (end 117.07 85.095) (width 1) (layer "B.Cu") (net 4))
 (segment (start 89.97 101.355) (end 92.72 101.355) (width 2) (layer "B.Cu") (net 4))
 (segment (start 98.72 109.855) (end 98.72 98.855) (width 2) (layer "B.Cu") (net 4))
 (segment (start 95.1 101.355) (end 96.41 102.665) (width 2) (layer "B.Cu") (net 4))
 (segment (start 98.8675 111.4575) (end 99.87 110.455) (width 2) (layer "B.Cu") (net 4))
 (segment (start 98.72 98.855) (end 98.66 98.795) (width 2) (layer "B.Cu") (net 4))
 (segment (start 96.97 89.54) (end 96.97 87.605) (width 2) (layer "B.Cu") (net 4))
 (segment (start 88.22 100.105) (end 92.22 100.105) (width 2) (layer "B.Cu") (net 4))
 (segment (start 97.1 111.4575) (end 98.8675 111.4575) (width 2) (layer "B.Cu") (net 4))
 (segment (start 96.41 102.665) (end 97.1 103.355) (width 2) (layer "B.Cu") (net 4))
 (segment (start 116.45 84.475) (end 112.95 84.475) (width 1) (layer "B.Cu") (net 4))
 (segment (start 97.0025 94.855) (end 97.0025 89.5725) (width 2) (layer "B.Cu") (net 4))
 (segment (start 99.87 87.365) (end 99.87 88.605) (width 2) (layer "B.Cu") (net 4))
 (segment (start 116.01 103.395) (end 115.97 103.355) (width 1) (layer "B.Cu") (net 1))
 (segment (start 115.97 103.355) (end 117.01 102.315) (width 1) (layer "B.Cu") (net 1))
 (segment (start 116.01 107.775) (end 116.01 103.395) (width 1) (layer "B.Cu") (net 1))
 (segment (start 114.53 94.735) (end 114.53 98.415) (width 1) (layer "B.Cu") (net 1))
 (segment (start 114.53 98.415) (end 115.47 99.355) (width 1) (layer "B.Cu") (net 1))
 (segment (start 115.47 99.355) (end 117.01 99.355) (width 1) (layer "B.Cu") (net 1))
 (segment (start 117.01 102.315) (end 117.01 99.355) (width 1) (layer "B.Cu") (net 1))
 (segment (start 73.68 86.895) (end 74.47 86.105) (width 2) (layer "B.Cu") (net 3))
 (segment (start 73.68 88.065) (end 73.68 86.895) (width 2) (layer "B.Cu") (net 3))
 (segment (start 78.47 86.105) (end 78.47 88.605) (width 2) (layer "B.Cu") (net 3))
 (segment (start 78.47 88.605) (end 74.22 88.605) (width 2) (layer "B.Cu") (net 3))
 (segment (start 73.68 87.365) (end 78.03 87.365) (width 2) (layer "B.Cu") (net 3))
 (segment (start 73.68 88.065) (end 73.68 87.365) (width 2) (layer "B.Cu") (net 3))
 (segment (start 74.22 88.605) (end 73.68 88.065) (width 2) (layer "B.Cu") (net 3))
 (segment (start 74.47 86.105) (end 78.47 86.105) (width 2) (layer "B.Cu") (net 3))
 (segment (start 108.72 108.355) (end 108.72 98.355) (width 1) (layer "B.Cu") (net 6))
 (segment (start 108.72 90.855) (end 113.07 90.855) (width 1) (layer "B.Cu") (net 6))
 (segment (start 108.72 98.355) (end 108.72 90.855) (width 1) (layer "B.Cu") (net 6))
 (segment (start 107.63 99.695) (end 108.72 98.605) (width 1) (layer "B.Cu") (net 6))
 (segment (start 114.53 89.395) (end 114.53 87.115) (width 1) (layer "B.Cu") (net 6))
 (segment (start 113.07 90.855) (end 114.53 89.395) (width 1) (layer "B.Cu") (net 6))
 (segment (start 105.62 99.695) (end 107.63 99.695) (width 1) (layer "B.Cu") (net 6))
 (segment (start 105.62 109.445) (end 107.63 109.445) (width 1) (layer "B.Cu") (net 6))
 (segment (start 107.81 89.945) (end 108.72 90.855) (width 1) (layer "B.Cu") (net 6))
 (segment (start 107.63 109.445) (end 108.72 108.355) (width 1) (layer "B.Cu") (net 6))
 (segment (start 105.62 89.945) (end 107.81 89.945) (width 1) (layer "B.Cu") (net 6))
 (segment (start 108.72 98.605) (end 108.72 98.355) (width 0.5) (layer "B.Cu") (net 6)))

